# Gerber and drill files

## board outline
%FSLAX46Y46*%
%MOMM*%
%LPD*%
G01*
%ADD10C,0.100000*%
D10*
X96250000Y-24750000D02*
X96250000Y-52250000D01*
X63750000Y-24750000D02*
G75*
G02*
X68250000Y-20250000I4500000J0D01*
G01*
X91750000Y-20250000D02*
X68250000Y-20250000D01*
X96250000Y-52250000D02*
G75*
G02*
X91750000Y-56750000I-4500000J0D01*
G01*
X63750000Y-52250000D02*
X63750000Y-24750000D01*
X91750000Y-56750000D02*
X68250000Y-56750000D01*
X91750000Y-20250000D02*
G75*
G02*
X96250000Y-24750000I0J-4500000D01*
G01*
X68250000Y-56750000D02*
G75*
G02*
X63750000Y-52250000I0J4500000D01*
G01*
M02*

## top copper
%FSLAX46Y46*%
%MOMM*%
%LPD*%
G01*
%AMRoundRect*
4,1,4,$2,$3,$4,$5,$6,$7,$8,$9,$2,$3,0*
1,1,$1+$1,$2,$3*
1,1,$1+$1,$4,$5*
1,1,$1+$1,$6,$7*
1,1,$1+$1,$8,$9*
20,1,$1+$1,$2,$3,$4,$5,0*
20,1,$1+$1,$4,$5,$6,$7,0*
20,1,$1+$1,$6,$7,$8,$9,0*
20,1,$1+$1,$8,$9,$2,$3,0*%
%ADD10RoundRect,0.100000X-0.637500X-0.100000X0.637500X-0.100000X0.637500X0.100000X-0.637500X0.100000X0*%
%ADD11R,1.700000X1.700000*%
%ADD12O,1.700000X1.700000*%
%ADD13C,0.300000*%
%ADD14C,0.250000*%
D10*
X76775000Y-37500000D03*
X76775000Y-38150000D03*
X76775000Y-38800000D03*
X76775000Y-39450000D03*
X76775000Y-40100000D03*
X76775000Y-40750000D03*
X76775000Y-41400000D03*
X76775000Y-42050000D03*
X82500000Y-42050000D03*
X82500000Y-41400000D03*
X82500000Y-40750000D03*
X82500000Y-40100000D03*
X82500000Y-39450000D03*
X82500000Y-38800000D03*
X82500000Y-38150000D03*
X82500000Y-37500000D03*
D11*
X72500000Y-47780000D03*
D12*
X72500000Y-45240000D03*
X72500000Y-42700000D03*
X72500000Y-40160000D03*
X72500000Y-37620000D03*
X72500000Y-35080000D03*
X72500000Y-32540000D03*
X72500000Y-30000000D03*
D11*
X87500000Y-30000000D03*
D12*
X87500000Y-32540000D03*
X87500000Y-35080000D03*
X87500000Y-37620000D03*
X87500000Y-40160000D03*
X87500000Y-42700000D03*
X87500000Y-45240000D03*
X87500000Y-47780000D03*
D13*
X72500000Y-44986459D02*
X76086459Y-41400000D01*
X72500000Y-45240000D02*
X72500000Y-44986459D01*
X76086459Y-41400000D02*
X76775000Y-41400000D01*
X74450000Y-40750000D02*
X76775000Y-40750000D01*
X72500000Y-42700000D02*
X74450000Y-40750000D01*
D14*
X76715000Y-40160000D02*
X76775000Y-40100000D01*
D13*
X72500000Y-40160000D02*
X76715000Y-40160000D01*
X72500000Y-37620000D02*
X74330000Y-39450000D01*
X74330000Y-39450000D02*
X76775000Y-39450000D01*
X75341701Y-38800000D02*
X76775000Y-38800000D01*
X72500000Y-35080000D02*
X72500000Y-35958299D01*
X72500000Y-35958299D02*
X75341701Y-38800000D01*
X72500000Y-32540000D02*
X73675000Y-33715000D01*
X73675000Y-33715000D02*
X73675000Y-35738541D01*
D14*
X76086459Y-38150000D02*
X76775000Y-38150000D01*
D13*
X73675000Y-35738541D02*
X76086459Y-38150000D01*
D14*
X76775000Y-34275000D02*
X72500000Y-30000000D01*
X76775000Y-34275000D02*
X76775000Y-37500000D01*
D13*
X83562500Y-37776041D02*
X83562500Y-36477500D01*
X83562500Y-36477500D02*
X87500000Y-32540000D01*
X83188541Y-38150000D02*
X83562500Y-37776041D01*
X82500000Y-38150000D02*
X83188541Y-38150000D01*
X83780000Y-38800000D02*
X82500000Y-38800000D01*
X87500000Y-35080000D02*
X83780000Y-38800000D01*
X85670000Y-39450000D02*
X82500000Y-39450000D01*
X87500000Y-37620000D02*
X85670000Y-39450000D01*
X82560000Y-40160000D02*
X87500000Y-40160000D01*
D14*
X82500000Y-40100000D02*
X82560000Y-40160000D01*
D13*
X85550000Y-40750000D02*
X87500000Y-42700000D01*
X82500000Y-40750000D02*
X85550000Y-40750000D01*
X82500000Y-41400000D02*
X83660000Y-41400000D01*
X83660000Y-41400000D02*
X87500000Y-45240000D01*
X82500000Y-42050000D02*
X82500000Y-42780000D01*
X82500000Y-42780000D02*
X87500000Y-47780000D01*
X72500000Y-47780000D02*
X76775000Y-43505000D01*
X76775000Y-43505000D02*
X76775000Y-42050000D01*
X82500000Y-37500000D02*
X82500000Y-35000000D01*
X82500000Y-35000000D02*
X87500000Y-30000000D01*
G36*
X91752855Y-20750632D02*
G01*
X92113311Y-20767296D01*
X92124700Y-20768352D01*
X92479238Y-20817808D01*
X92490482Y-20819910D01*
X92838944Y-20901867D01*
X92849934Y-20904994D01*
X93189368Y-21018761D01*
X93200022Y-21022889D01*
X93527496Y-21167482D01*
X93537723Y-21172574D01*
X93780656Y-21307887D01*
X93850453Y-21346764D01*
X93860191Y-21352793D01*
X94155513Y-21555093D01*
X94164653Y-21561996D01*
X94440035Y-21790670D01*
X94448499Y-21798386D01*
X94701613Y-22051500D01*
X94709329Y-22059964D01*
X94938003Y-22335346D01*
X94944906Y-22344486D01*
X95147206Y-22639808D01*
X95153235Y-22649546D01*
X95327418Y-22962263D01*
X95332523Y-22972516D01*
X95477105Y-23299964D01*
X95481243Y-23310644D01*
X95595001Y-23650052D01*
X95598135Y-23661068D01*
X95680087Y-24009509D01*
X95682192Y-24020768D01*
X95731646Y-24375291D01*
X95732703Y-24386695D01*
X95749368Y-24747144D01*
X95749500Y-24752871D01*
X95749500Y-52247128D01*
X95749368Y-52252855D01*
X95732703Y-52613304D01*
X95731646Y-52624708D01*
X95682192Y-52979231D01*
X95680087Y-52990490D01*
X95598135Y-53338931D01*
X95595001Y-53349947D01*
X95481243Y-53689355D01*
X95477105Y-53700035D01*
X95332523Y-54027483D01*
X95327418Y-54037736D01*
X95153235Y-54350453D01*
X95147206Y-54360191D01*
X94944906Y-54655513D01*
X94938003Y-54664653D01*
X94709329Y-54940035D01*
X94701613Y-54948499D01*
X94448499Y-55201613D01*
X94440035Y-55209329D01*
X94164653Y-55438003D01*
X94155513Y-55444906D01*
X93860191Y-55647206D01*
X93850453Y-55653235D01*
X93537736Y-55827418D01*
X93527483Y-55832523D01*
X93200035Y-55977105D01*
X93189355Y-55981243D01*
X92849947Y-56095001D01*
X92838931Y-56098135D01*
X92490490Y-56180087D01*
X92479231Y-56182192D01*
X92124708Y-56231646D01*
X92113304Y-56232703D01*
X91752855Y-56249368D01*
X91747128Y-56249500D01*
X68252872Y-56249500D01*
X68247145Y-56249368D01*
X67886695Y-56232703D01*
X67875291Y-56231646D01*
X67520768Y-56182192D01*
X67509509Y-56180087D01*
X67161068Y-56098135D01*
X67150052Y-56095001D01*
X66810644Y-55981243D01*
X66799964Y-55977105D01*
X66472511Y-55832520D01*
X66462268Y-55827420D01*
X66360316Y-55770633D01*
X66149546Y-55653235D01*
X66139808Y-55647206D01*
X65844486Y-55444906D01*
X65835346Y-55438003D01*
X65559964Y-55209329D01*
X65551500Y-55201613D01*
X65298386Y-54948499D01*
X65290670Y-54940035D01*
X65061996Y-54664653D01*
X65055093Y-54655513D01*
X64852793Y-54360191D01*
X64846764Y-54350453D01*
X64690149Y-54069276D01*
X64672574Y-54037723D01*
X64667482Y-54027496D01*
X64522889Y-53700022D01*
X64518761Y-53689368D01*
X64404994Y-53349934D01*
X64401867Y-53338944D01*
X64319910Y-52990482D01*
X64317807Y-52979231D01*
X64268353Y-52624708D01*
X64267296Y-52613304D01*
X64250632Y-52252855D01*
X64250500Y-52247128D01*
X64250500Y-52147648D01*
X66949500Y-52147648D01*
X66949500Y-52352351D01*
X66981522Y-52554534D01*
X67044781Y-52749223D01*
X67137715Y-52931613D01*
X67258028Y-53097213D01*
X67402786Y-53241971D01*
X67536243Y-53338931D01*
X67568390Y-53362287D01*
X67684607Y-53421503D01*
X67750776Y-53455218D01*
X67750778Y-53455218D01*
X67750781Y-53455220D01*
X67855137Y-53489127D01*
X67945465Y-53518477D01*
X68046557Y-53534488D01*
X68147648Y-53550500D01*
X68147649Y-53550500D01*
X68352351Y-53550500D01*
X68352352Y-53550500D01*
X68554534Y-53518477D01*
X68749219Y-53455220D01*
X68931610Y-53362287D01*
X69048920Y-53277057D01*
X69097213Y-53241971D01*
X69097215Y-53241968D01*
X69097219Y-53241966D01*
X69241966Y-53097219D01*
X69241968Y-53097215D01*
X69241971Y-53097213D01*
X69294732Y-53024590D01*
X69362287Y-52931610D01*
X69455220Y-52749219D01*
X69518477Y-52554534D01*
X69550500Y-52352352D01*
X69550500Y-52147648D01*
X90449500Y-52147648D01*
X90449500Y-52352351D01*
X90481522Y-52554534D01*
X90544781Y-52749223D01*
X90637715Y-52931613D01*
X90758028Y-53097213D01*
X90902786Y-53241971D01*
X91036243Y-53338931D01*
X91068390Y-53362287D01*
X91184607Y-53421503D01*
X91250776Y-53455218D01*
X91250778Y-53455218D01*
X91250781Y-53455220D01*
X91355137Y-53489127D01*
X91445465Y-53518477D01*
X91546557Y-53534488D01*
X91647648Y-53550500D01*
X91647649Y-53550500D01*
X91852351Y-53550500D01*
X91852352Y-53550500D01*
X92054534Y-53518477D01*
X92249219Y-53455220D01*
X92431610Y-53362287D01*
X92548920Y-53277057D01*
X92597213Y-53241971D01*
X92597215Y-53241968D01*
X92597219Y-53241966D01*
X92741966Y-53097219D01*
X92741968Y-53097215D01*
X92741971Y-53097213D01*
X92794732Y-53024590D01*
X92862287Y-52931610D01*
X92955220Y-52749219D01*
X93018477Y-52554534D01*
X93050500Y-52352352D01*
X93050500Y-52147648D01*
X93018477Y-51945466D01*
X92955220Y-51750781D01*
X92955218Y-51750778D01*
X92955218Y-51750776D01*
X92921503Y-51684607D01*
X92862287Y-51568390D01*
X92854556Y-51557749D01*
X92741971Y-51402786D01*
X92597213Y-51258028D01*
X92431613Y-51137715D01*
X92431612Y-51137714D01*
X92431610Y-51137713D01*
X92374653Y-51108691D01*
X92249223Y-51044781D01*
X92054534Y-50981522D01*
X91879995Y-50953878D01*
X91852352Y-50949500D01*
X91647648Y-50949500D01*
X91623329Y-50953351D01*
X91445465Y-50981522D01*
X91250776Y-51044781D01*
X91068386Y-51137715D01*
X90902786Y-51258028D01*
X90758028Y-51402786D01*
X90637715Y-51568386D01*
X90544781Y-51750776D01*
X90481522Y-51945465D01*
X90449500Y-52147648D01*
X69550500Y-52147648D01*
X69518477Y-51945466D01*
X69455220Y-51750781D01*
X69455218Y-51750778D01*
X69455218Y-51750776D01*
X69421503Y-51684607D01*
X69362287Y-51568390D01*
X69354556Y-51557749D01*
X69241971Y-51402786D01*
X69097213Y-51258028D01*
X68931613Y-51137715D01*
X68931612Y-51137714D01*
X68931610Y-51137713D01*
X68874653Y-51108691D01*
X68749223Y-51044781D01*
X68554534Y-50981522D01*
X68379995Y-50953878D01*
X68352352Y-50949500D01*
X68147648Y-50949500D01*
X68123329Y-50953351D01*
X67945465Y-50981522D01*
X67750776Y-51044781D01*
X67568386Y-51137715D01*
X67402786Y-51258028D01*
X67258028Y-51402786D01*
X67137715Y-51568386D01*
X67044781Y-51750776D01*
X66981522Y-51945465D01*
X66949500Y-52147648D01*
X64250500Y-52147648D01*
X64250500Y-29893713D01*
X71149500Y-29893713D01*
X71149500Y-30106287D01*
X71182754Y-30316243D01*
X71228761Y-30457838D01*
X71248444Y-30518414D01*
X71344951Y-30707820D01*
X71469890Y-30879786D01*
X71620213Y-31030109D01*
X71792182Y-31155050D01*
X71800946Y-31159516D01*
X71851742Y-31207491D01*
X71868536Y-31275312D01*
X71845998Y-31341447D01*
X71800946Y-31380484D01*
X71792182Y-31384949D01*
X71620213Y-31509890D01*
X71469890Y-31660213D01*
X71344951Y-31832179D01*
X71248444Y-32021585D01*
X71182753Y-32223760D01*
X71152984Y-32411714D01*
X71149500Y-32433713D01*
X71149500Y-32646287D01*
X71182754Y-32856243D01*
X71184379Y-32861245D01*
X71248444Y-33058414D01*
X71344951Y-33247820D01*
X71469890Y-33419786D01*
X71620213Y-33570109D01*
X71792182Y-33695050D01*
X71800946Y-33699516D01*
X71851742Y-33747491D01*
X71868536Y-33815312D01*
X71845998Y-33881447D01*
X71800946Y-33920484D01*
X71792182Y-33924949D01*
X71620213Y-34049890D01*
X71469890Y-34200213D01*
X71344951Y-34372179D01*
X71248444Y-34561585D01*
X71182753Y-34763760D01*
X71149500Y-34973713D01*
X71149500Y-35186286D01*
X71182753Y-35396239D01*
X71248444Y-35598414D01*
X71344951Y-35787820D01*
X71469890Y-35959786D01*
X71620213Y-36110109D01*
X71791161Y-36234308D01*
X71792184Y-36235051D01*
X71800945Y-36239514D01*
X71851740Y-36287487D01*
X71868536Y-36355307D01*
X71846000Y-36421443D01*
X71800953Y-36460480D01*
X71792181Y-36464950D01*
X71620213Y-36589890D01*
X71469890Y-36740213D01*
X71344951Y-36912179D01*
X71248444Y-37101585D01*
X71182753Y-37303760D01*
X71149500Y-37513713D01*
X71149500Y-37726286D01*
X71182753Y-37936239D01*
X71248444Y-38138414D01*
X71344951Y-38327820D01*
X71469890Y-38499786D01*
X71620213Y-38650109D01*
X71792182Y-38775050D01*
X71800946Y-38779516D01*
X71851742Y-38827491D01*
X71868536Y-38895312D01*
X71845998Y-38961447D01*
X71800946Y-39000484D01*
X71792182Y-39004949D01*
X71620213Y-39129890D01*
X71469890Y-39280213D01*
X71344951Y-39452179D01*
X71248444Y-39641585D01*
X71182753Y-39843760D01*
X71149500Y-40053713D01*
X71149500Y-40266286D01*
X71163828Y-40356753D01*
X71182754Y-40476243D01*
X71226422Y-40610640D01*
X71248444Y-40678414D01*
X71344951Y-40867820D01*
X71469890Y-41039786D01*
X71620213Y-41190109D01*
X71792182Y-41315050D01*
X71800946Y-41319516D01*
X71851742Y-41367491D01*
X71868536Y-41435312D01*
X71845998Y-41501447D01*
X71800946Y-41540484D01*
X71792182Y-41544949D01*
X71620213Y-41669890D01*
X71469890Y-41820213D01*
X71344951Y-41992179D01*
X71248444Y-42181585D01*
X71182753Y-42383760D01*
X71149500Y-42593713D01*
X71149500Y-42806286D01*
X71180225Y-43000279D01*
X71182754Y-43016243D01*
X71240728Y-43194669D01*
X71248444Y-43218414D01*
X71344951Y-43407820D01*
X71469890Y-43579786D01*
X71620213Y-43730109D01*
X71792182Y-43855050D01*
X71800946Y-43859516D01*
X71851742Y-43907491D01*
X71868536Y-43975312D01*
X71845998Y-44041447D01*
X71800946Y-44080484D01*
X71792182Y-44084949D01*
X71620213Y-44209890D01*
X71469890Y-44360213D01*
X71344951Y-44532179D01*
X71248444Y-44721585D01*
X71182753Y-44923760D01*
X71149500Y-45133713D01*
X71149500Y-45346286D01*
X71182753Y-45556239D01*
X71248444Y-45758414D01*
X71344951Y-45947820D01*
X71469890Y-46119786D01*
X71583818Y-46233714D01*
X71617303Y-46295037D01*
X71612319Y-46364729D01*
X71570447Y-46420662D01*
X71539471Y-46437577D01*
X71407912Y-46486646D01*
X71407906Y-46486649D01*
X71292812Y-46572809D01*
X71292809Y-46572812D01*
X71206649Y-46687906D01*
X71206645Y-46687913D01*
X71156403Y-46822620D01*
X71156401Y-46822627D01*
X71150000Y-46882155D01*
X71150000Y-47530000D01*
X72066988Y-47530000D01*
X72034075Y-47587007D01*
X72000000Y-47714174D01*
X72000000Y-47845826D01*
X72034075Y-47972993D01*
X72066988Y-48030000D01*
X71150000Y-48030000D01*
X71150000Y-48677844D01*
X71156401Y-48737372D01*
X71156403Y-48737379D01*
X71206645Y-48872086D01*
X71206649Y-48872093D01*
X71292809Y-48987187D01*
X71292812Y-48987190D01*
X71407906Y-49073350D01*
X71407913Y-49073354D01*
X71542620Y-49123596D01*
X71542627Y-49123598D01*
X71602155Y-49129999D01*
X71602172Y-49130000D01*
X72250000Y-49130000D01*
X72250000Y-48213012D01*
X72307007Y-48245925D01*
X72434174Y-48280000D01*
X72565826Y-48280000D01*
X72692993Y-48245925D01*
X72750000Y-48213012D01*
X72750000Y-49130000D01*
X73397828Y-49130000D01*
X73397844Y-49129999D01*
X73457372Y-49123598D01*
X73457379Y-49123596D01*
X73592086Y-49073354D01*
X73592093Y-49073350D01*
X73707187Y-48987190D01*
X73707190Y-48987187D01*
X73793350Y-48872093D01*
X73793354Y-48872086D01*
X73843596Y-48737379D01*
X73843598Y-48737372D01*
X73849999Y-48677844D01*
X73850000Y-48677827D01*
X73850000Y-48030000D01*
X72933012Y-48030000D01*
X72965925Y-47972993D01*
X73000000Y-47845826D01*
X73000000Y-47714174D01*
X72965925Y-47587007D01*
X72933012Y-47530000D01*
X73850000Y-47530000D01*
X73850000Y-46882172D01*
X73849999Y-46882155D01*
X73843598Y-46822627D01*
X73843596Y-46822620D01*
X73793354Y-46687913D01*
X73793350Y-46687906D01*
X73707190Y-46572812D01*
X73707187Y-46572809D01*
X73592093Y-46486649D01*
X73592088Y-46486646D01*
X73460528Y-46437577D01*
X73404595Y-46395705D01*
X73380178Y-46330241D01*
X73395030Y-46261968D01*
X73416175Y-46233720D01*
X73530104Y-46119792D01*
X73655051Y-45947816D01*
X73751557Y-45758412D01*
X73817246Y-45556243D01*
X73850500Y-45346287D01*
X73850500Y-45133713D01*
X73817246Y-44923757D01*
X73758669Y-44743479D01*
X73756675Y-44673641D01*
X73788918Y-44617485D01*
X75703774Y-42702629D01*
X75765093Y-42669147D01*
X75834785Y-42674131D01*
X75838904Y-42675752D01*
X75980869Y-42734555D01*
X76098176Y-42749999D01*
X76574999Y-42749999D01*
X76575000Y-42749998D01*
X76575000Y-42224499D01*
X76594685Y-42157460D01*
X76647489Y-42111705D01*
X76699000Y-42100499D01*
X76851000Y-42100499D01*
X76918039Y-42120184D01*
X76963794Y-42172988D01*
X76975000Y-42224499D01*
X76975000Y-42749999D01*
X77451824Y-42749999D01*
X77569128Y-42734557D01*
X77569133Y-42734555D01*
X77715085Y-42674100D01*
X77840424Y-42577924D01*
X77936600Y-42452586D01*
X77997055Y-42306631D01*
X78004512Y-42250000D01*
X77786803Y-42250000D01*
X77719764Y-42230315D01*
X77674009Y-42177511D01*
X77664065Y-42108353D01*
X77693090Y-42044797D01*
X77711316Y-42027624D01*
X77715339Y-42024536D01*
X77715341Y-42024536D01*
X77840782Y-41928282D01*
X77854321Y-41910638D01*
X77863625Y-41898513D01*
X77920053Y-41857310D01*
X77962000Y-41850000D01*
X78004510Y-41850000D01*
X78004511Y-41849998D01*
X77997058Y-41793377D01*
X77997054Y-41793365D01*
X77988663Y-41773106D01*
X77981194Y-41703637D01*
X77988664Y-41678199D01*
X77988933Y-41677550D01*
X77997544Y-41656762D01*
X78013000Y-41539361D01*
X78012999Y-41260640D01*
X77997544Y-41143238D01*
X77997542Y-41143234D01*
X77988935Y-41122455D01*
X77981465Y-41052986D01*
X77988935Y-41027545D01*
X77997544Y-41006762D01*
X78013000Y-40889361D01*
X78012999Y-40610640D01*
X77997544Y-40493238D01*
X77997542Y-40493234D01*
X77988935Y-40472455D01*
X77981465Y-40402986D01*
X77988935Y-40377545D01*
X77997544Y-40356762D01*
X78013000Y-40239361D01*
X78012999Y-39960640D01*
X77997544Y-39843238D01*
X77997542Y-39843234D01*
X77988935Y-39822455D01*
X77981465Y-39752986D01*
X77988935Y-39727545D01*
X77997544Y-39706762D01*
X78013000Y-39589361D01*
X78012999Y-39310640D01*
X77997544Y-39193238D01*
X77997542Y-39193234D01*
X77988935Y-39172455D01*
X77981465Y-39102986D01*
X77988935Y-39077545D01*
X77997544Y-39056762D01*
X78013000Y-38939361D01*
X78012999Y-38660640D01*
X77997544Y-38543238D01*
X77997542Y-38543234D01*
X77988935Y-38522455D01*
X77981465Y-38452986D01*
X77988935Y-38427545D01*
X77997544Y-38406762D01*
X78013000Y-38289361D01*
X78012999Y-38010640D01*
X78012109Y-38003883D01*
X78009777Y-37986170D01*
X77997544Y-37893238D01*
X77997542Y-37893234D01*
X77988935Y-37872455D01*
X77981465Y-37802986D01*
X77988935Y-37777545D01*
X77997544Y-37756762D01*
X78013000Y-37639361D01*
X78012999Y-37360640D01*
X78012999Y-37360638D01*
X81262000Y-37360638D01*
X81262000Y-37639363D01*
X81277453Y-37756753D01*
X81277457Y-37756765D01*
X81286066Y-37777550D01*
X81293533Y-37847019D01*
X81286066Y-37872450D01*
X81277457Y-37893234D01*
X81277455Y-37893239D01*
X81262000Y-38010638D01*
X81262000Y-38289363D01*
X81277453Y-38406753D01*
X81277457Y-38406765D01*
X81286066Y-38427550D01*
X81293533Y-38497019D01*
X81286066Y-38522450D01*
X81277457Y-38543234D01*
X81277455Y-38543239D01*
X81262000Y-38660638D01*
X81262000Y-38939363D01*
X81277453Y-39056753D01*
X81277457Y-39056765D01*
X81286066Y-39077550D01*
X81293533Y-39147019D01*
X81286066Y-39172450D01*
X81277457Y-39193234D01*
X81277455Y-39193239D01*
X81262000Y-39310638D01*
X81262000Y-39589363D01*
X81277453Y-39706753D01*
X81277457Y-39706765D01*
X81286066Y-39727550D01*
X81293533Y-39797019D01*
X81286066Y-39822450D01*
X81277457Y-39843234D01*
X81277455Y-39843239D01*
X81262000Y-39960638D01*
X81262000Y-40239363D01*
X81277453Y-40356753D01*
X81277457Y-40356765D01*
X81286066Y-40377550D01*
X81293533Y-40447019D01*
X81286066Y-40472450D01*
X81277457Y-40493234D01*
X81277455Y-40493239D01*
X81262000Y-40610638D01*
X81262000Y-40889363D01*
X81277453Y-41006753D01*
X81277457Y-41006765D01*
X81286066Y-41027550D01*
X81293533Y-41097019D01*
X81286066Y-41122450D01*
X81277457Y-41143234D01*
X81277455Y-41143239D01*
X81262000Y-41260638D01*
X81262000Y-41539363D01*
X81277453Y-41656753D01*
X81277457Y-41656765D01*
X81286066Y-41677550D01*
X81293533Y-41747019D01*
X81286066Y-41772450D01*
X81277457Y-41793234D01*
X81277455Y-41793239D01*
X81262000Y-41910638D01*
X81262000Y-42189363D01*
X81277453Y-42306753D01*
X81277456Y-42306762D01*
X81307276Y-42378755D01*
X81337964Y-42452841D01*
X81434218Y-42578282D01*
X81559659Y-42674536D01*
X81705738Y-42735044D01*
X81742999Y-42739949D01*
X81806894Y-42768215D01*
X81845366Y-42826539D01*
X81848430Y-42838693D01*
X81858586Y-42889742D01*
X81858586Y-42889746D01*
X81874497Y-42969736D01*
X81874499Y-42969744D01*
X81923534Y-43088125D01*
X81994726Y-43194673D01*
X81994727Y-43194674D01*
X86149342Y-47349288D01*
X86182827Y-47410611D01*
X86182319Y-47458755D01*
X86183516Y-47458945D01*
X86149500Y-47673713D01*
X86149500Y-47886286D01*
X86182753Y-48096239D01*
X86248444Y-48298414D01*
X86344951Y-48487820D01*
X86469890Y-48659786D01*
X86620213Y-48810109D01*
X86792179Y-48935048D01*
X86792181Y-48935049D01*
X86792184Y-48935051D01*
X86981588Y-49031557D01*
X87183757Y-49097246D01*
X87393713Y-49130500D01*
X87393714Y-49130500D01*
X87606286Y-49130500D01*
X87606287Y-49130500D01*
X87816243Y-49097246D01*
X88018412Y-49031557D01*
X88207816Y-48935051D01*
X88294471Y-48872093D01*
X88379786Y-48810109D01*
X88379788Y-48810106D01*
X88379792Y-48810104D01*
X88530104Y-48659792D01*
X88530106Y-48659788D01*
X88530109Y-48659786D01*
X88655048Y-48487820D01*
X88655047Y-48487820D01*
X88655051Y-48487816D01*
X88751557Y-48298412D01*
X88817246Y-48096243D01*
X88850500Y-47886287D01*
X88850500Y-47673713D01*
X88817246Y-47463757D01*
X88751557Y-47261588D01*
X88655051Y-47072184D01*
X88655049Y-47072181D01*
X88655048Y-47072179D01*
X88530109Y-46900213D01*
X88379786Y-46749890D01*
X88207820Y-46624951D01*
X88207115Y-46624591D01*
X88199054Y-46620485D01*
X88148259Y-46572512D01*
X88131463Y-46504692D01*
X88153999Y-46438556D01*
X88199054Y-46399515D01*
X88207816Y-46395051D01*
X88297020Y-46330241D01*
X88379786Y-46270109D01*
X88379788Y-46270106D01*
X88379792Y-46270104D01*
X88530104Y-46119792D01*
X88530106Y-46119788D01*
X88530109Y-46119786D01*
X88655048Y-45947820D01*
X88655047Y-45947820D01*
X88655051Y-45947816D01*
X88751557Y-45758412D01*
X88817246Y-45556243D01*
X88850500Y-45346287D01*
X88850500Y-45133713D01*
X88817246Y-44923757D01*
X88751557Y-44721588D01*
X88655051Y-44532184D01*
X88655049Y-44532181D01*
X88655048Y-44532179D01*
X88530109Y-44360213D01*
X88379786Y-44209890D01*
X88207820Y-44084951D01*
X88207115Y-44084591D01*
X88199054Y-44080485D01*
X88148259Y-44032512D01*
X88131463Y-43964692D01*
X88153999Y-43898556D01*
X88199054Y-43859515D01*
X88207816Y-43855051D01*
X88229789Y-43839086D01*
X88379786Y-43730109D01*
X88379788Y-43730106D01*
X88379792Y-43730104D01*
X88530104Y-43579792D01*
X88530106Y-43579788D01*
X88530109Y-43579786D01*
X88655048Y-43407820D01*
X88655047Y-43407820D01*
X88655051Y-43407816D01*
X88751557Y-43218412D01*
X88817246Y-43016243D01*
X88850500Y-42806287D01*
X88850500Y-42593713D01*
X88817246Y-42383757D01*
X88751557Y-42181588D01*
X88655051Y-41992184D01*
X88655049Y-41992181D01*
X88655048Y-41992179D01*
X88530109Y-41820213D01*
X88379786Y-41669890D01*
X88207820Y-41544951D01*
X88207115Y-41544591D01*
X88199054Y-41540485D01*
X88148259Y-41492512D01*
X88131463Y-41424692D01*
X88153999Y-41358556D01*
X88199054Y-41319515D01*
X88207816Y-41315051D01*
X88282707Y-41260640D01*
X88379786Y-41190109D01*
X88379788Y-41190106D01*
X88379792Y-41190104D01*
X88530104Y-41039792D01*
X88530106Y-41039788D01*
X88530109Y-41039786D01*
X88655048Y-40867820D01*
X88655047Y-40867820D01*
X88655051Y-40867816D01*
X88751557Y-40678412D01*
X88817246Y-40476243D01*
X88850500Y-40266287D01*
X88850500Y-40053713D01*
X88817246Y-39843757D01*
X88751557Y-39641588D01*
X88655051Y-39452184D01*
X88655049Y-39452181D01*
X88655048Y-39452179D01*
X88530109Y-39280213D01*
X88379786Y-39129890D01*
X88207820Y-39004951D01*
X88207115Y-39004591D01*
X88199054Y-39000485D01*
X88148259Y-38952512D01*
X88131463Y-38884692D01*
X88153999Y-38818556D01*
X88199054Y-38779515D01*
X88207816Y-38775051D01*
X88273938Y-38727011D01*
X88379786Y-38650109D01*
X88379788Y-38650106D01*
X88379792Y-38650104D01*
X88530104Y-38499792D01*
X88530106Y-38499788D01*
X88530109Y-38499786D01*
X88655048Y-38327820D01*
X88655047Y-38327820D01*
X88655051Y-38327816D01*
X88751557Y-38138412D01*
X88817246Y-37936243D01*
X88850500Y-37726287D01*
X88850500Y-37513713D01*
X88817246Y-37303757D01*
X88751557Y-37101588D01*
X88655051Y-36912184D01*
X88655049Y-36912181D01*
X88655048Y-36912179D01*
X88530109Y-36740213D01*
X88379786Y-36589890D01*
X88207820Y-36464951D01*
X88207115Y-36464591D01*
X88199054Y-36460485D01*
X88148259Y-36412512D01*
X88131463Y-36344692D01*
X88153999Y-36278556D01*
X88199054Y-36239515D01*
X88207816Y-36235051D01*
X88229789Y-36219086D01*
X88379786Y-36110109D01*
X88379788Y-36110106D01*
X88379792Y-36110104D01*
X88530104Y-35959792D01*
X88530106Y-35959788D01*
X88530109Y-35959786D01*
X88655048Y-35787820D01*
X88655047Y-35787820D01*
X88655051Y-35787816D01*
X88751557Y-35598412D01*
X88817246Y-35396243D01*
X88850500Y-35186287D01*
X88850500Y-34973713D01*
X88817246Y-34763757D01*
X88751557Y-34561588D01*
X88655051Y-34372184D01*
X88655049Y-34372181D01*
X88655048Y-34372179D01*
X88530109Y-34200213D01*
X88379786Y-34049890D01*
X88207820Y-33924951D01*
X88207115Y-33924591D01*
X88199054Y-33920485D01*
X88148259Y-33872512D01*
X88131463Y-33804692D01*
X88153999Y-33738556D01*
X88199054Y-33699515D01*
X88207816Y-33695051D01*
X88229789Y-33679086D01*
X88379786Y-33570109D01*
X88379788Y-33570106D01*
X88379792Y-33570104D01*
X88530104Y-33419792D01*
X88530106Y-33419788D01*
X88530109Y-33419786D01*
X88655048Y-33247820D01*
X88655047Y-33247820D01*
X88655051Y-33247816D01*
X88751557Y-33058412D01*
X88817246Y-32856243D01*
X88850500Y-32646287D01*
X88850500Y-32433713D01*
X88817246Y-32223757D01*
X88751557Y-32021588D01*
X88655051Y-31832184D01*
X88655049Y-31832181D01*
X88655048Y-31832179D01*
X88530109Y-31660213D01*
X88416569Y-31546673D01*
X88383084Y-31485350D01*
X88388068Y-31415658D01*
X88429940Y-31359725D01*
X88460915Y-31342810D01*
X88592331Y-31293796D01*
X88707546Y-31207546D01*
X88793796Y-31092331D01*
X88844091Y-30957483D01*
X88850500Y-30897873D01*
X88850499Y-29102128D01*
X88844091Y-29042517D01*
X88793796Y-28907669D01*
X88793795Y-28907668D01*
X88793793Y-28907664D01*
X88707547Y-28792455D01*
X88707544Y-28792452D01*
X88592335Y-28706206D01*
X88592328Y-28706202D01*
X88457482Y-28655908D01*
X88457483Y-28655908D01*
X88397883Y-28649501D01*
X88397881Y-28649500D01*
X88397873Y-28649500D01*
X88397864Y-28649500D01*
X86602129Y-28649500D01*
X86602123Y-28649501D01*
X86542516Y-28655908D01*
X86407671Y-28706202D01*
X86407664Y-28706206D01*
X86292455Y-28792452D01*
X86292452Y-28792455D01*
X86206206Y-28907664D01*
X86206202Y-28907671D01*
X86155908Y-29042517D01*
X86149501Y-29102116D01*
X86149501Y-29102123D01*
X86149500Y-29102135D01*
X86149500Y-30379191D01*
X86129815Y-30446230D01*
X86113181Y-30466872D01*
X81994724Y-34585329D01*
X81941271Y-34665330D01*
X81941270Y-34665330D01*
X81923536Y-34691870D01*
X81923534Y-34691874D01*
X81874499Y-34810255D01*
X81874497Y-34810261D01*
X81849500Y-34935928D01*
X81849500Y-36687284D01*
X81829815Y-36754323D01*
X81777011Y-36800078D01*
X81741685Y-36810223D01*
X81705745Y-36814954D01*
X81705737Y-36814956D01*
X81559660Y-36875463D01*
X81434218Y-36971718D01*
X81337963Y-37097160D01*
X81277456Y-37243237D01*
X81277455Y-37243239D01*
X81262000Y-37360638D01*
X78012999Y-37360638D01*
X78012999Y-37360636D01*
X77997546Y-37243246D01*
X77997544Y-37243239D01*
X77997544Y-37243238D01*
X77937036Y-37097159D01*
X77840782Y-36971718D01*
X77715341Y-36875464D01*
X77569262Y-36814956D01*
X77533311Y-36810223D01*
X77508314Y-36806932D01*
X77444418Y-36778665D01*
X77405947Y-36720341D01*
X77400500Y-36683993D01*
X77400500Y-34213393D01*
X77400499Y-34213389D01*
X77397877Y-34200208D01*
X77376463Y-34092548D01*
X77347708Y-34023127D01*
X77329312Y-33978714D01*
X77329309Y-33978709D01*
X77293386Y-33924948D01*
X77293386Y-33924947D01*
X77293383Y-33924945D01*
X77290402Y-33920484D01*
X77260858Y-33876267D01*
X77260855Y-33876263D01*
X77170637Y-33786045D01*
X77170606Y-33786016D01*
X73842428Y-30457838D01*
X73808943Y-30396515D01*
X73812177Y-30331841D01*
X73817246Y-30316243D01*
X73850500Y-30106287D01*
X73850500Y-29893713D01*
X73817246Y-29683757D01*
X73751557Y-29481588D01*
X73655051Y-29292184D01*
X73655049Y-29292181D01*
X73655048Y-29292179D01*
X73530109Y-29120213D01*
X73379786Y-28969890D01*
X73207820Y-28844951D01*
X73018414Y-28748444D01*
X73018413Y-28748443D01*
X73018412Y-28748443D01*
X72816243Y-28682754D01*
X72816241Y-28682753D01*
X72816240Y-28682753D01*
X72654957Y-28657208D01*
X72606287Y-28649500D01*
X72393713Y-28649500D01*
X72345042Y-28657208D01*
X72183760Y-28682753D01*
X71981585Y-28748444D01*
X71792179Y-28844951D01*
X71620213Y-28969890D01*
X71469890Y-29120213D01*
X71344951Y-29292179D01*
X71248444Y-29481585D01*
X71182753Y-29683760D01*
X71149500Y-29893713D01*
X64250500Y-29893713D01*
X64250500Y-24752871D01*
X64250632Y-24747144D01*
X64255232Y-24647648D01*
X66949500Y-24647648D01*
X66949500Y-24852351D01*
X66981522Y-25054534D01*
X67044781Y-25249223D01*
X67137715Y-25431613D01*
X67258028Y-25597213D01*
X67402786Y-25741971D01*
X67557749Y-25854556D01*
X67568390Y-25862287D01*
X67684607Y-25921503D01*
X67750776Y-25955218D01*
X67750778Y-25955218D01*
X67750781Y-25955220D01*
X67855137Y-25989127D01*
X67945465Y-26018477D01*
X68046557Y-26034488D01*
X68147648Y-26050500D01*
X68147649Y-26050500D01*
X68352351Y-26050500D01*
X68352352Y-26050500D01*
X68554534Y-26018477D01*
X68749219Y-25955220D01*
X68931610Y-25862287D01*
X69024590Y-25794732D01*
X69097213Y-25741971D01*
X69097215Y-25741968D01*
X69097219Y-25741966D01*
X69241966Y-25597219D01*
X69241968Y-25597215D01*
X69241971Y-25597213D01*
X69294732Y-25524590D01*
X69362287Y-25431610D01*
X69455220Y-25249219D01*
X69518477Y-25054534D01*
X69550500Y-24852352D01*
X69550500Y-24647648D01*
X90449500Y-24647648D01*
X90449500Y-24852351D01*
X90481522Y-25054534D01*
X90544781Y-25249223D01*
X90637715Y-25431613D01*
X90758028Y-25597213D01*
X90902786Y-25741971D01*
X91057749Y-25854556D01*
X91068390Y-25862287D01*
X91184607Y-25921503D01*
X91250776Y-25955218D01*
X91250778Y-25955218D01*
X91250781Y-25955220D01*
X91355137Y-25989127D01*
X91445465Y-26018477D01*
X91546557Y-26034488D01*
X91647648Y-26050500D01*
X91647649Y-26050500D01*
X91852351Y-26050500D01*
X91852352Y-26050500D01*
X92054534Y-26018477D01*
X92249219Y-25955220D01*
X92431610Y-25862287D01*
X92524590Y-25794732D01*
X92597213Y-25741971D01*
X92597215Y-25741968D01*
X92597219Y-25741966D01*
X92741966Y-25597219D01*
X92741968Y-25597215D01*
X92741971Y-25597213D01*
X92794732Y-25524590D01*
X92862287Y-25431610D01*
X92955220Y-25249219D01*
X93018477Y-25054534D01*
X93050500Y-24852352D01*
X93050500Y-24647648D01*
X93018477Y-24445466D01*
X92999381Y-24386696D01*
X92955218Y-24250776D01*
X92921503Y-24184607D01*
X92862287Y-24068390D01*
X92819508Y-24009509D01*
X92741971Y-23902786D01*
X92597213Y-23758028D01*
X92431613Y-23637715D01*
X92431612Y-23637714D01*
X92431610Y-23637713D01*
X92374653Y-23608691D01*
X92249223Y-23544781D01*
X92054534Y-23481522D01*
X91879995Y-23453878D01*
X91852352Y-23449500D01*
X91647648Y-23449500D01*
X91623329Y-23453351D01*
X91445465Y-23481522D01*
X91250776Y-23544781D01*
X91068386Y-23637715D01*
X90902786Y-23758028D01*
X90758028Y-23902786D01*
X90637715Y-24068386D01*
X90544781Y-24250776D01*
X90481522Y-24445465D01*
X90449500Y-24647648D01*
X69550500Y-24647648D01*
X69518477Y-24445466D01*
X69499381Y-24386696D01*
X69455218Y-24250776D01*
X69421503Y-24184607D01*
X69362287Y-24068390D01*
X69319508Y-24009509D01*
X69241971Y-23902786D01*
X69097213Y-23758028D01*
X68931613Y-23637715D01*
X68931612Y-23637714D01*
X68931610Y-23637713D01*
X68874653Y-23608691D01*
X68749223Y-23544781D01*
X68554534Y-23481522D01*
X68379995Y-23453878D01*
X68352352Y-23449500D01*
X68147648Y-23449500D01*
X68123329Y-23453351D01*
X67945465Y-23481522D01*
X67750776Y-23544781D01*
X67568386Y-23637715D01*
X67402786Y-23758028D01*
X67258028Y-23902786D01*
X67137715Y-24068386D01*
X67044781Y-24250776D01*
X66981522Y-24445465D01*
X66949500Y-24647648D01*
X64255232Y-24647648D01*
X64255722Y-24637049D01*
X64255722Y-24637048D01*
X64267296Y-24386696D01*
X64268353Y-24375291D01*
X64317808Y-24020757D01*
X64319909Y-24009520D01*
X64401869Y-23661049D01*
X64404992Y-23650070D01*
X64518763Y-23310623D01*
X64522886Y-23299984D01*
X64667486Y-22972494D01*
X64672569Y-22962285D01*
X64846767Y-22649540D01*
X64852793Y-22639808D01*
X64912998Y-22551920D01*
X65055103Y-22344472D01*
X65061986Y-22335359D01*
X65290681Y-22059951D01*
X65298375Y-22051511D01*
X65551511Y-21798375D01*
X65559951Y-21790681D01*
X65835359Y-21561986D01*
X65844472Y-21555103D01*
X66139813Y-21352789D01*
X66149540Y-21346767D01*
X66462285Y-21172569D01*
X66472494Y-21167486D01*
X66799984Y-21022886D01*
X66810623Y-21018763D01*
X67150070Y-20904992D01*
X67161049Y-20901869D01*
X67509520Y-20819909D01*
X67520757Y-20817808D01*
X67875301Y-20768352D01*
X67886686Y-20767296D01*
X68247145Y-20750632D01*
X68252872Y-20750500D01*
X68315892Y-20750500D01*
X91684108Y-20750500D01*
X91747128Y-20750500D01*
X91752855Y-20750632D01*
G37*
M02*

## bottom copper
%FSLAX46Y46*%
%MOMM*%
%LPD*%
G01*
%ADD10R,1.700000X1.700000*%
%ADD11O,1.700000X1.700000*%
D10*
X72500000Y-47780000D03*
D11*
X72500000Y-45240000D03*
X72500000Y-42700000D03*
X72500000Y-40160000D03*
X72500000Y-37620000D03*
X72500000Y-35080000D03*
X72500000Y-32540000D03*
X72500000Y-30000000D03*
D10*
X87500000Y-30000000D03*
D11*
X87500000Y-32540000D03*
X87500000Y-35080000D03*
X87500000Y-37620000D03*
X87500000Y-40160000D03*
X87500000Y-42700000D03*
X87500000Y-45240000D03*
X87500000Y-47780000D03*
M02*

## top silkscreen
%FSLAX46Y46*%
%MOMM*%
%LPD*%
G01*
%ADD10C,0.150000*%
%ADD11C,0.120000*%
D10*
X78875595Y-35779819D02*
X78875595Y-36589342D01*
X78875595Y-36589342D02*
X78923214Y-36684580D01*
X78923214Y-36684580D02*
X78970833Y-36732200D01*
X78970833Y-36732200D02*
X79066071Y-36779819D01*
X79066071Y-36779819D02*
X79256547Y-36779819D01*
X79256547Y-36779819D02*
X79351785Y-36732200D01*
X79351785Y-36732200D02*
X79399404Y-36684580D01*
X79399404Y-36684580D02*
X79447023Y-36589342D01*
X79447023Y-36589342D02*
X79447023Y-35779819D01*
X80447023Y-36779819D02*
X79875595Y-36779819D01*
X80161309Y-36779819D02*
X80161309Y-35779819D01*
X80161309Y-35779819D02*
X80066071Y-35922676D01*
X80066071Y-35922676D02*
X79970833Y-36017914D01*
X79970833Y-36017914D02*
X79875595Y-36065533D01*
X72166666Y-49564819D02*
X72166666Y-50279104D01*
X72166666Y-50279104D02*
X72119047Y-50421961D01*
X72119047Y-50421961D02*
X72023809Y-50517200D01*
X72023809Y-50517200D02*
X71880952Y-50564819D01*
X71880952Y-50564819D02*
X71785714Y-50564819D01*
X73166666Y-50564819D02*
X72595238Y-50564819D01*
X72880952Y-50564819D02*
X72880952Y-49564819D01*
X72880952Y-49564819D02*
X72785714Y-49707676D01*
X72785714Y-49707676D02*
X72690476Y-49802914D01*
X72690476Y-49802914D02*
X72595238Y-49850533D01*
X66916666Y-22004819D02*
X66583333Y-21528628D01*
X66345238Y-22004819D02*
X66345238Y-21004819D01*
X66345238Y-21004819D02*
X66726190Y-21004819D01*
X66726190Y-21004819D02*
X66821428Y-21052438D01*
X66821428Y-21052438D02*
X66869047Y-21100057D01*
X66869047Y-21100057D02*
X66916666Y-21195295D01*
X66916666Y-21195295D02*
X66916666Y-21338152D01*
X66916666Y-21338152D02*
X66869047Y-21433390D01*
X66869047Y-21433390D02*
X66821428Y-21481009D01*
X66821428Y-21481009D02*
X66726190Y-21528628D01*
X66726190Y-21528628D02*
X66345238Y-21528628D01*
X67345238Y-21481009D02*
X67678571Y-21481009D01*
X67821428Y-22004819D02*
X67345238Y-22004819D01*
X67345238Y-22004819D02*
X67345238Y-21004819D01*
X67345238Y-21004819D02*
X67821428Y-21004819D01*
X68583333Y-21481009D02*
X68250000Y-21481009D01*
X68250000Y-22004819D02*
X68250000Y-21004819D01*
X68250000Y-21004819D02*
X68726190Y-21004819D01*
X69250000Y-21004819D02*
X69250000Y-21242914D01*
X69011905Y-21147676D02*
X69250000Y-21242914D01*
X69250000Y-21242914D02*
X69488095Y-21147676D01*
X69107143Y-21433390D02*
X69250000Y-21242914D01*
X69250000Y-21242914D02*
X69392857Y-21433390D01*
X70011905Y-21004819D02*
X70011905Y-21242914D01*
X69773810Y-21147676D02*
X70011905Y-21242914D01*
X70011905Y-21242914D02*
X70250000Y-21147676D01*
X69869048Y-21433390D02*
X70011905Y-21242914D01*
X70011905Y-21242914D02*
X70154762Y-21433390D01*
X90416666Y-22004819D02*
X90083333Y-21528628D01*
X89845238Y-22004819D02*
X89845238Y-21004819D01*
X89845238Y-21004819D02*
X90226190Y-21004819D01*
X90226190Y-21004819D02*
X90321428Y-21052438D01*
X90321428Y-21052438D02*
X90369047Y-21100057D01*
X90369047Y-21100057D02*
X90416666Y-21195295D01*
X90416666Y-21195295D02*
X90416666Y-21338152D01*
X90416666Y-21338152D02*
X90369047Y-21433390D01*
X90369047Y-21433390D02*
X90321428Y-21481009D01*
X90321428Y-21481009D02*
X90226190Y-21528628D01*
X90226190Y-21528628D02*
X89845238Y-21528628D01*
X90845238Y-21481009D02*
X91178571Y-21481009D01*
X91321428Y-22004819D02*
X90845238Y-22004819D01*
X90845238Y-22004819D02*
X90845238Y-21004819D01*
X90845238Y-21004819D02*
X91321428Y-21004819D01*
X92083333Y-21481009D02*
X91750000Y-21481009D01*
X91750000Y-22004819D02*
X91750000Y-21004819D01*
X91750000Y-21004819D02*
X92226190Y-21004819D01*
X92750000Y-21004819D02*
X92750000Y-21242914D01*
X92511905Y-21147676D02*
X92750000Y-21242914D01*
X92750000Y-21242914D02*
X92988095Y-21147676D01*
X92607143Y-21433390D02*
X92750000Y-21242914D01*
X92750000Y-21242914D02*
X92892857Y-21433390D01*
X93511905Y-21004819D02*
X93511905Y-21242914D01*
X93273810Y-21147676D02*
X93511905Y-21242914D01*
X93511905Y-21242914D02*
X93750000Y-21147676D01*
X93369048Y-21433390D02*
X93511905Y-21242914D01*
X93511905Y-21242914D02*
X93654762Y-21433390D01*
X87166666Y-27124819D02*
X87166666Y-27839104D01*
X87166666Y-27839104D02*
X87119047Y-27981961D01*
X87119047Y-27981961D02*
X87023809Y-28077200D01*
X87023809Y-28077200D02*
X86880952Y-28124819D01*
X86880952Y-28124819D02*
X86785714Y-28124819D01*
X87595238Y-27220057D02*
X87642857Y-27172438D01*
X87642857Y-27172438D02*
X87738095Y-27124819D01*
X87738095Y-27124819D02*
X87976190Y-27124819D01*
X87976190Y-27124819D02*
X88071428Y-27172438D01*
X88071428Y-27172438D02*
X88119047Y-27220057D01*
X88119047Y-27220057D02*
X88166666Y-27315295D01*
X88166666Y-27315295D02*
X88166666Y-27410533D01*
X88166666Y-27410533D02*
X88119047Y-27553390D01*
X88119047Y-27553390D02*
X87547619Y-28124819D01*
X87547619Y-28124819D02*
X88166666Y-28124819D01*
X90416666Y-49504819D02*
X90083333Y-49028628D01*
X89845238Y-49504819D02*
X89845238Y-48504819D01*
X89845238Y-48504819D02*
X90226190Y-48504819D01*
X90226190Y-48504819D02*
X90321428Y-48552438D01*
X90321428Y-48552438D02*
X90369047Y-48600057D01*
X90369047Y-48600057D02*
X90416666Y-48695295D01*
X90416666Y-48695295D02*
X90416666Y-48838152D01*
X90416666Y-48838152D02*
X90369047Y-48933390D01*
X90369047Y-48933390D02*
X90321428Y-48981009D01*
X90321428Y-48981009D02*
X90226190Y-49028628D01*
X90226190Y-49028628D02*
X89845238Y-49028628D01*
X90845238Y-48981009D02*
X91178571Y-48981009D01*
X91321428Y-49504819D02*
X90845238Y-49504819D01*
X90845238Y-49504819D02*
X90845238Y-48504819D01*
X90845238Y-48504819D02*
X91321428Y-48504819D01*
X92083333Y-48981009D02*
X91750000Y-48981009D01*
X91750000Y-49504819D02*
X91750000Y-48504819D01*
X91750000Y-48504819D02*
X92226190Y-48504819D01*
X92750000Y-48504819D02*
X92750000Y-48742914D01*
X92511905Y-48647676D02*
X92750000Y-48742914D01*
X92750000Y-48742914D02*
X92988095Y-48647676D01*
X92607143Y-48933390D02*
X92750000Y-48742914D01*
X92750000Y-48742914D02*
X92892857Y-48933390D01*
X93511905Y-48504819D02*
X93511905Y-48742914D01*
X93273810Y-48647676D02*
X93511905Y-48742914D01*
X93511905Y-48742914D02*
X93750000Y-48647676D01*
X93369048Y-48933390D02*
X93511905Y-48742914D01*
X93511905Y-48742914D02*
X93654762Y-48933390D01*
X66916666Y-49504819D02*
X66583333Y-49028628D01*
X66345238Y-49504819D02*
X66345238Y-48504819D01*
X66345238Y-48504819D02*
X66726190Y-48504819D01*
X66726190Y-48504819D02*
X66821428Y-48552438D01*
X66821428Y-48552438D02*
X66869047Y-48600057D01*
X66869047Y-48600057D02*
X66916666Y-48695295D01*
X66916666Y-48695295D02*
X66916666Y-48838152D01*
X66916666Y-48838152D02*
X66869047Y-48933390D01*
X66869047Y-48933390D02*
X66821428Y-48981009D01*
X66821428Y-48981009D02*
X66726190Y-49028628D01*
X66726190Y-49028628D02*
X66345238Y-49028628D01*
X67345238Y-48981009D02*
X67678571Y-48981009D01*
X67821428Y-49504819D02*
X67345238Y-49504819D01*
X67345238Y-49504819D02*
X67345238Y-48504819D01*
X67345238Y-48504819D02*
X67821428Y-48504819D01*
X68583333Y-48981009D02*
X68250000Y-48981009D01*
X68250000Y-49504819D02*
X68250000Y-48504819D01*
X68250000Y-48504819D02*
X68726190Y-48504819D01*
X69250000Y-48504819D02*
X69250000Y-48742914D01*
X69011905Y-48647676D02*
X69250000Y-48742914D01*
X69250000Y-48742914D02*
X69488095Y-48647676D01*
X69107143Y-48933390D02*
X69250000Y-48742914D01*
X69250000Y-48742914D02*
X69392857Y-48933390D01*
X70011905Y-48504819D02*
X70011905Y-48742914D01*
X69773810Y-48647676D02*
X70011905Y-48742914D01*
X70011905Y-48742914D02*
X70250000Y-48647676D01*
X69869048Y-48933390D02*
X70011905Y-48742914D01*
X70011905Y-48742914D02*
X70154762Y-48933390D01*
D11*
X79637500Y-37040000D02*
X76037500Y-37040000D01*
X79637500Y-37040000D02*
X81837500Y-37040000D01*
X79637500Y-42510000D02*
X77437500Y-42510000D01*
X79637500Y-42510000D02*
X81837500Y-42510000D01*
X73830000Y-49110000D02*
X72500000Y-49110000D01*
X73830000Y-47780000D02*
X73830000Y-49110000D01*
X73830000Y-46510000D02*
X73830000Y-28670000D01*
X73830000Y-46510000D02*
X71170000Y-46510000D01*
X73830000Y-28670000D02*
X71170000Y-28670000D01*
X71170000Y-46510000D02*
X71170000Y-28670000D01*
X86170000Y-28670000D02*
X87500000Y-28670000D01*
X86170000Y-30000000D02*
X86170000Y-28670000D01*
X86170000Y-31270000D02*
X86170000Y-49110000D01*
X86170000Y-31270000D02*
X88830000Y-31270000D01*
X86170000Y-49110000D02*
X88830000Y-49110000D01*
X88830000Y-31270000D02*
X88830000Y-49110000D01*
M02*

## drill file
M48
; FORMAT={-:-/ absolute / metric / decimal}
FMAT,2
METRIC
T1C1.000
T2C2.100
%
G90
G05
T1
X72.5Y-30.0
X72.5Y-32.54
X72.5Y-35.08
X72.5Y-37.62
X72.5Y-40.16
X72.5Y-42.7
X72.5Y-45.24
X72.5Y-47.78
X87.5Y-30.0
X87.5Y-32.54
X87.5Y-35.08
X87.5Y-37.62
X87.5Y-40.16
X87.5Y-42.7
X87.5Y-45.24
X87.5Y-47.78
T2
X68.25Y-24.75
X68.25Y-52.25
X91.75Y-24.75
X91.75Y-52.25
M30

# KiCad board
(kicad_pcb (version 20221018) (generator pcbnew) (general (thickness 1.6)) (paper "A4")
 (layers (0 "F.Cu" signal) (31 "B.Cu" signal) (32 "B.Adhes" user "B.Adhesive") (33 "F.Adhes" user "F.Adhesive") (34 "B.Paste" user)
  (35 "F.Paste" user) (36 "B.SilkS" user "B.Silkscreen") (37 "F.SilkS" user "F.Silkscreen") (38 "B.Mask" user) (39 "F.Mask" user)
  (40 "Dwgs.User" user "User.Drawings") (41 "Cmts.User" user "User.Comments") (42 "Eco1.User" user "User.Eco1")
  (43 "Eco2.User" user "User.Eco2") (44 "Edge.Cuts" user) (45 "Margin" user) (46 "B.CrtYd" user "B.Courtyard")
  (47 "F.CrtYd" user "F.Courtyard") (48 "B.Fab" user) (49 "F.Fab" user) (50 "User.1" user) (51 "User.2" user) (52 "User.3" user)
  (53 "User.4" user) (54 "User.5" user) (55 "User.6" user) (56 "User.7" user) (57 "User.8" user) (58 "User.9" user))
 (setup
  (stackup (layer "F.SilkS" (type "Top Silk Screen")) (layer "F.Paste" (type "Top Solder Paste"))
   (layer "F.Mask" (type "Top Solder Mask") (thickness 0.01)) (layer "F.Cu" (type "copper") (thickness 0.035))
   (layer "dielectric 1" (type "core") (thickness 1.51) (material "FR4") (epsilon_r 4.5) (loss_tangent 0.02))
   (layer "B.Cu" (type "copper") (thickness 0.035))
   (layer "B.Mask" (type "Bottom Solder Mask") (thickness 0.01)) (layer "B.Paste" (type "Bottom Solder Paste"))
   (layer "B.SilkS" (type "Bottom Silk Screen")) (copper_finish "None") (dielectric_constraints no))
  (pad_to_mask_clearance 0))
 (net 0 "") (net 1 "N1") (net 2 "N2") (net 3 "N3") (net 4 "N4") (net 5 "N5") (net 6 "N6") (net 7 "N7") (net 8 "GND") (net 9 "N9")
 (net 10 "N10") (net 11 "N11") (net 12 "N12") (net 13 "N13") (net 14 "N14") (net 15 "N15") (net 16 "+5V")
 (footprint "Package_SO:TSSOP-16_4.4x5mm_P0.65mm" (layer "F.Cu") (at 79.6375 39.775)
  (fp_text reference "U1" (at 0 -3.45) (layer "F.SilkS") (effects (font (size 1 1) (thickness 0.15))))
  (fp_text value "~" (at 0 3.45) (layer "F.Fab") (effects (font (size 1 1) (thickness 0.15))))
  (fp_line (start 0 -2.735) (end -3.6 -2.735) (stroke (width 0.12) (type solid)) (layer "F.SilkS"))
  (fp_line (start 0 -2.735) (end 2.2 -2.735) (stroke (width 0.12) (type solid)) (layer "F.SilkS"))
  (fp_line (start 0 2.735) (end -2.2 2.735) (stroke (width 0.12) (type solid)) (layer "F.SilkS"))
  (fp_line (start 0 2.735) (end 2.2 2.735) (stroke (width 0.12) (type solid)) (layer "F.SilkS"))
  (pad "1" smd roundrect (at -2.8625 -2.275) (size 1.475 0.4) (layers "F.Cu" "F.Paste" "F.Mask") (roundrect_rratio 0.25) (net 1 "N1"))
  (pad "2" smd roundrect (at -2.8625 -1.625) (size 1.475 0.4) (layers "F.Cu" "F.Paste" "F.Mask") (roundrect_rratio 0.25) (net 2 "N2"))
  (pad "3" smd roundrect (at -2.8625 -0.975) (size 1.475 0.4) (layers "F.Cu" "F.Paste" "F.Mask") (roundrect_rratio 0.25) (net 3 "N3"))
  (pad "4" smd roundrect (at -2.8625 -0.325) (size 1.475 0.4) (layers "F.Cu" "F.Paste" "F.Mask") (roundrect_rratio 0.25) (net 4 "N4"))
  (pad "5" smd roundrect (at -2.8625 0.325) (size 1.475 0.4) (layers "F.Cu" "F.Paste" "F.Mask") (roundrect_rratio 0.25) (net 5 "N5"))
  (pad "6" smd roundrect (at -2.8625 0.975) (size 1.475 0.4) (layers "F.Cu" "F.Paste" "F.Mask") (roundrect_rratio 0.25) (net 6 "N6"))
  (pad "7" smd roundrect (at -2.8625 1.625) (size 1.475 0.4) (layers "F.Cu" "F.Paste" "F.Mask") (roundrect_rratio 0.25) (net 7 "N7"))
  (pad "8" smd roundrect (at -2.8625 2.275) (size 1.475 0.4) (layers "F.Cu" "F.Paste" "F.Mask") (roundrect_rratio 0.25) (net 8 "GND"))
  (pad "9" smd roundrect (at 2.8625 2.275) (size 1.475 0.4) (layers "F.Cu" "F.Paste" "F.Mask") (roundrect_rratio 0.25) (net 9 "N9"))
  (pad "10" smd roundrect (at 2.8625 1.625) (size 1.475 0.4) (layers "F.Cu" "F.Paste" "F.Mask") (roundrect_rratio 0.25) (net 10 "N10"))
  (pad "11" smd roundrect (at 2.8625 0.975) (size 1.475 0.4) (layers "F.Cu" "F.Paste" "F.Mask") (roundrect_rratio 0.25) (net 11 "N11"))
  (pad "12" smd roundrect (at 2.8625 0.325) (size 1.475 0.4) (layers "F.Cu" "F.Paste" "F.Mask") (roundrect_rratio 0.25) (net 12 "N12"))
  (pad "13" smd roundrect (at 2.8625 -0.325) (size 1.475 0.4) (layers "F.Cu" "F.Paste" "F.Mask") (roundrect_rratio 0.25) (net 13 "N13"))
  (pad "14" smd roundrect (at 2.8625 -0.975) (size 1.475 0.4) (layers "F.Cu" "F.Paste" "F.Mask") (roundrect_rratio 0.25) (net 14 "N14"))
  (pad "15" smd roundrect (at 2.8625 -1.625) (size 1.475 0.4) (layers "F.Cu" "F.Paste" "F.Mask") (roundrect_rratio 0.25) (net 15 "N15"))
  (pad "16" smd roundrect (at 2.8625 -2.275) (size 1.475 0.4) (layers "F.Cu" "F.Paste" "F.Mask") (roundrect_rratio 0.25) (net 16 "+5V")))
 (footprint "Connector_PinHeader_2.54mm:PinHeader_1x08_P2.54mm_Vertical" (layer "F.Cu") (at 72.5 47.78 180)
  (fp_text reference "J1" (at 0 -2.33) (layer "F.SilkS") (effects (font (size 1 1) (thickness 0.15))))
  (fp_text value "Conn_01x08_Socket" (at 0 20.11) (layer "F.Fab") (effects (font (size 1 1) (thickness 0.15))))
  (fp_line (start -1.33 -1.33) (end 0 -1.33) (stroke (width 0.12) (type solid)) (layer "F.SilkS"))
  (fp_line (start -1.33 0) (end -1.33 -1.33) (stroke (width 0.12) (type solid)) (layer "F.SilkS"))
  (fp_line (start -1.33 1.27) (end -1.33 19.11) (stroke (width 0.12) (type solid)) (layer "F.SilkS"))
  (fp_line (start -1.33 1.27) (end 1.33 1.27) (stroke (width 0.12) (type solid)) (layer "F.SilkS"))
  (fp_line (start -1.33 19.11) (end 1.33 19.11) (stroke (width 0.12) (type solid)) (layer "F.SilkS"))
  (fp_line (start 1.33 1.27) (end 1.33 19.11) (stroke (width 0.12) (type solid)) (layer "F.SilkS"))
  (pad "1" thru_hole rect (at 0 0 180) (size 1.7 1.7) (drill 1) (layers "*.Cu" "*.Mask") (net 8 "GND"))
  (pad "2" thru_hole oval (at 0 2.54 180) (size 1.7 1.7) (drill 1) (layers "*.Cu" "*.Mask") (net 7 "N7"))
  (pad "3" thru_hole oval (at 0 5.08 180) (size 1.7 1.7) (drill 1) (layers "*.Cu" "*.Mask") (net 6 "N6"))
  (pad "4" thru_hole oval (at 0 7.62 180) (size 1.7 1.7) (drill 1) (layers "*.Cu" "*.Mask") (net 5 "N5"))
  (pad "5" thru_hole oval (at 0 10.16 180) (size 1.7 1.7) (drill 1) (layers "*.Cu" "*.Mask") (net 4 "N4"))
  (pad "6" thru_hole oval (at 0 12.7 180) (size 1.7 1.7) (drill 1) (layers "*.Cu" "*.Mask") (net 3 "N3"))
  (pad "7" thru_hole oval (at 0 15.24 180) (size 1.7 1.7) (drill 1) (layers "*.Cu" "*.Mask") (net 2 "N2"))
  (pad "8" thru_hole oval (at 0 17.78 180) (size 1.7 1.7) (drill 1) (layers "*.Cu" "*.Mask") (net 1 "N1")))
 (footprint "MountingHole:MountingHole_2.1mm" (layer "F.Cu") (at 68.25 24.75)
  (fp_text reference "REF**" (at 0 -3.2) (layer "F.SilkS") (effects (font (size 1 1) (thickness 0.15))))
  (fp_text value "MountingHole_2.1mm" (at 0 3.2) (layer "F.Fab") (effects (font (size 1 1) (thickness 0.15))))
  (pad "" np_thru_hole circle (at 0 0) (size 2.1 2.1) (drill 2.1) (layers "*.Cu" "*.Mask")))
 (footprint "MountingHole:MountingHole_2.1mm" (layer "F.Cu") (at 91.75 24.75)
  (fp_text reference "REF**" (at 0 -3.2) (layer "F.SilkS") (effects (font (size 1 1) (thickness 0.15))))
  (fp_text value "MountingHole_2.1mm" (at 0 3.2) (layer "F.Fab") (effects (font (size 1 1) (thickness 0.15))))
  (pad "" np_thru_hole circle (at 0 0) (size 2.1 2.1) (drill 2.1) (layers "*.Cu" "*.Mask")))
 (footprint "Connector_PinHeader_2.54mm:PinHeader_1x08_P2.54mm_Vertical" (layer "F.Cu") (at 87.5 30)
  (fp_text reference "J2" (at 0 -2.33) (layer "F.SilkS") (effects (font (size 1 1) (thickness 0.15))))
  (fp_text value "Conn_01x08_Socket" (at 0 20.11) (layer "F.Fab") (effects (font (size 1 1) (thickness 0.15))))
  (fp_line (start -1.33 -1.33) (end 0 -1.33) (stroke (width 0.12) (type solid)) (layer "F.SilkS"))
  (fp_line (start -1.33 0) (end -1.33 -1.33) (stroke (width 0.12) (type solid)) (layer "F.SilkS"))
  (fp_line (start -1.33 1.27) (end -1.33 19.11) (stroke (width 0.12) (type solid)) (layer "F.SilkS"))
  (fp_line (start -1.33 1.27) (end 1.33 1.27) (stroke (width 0.12) (type solid)) (layer "F.SilkS"))
  (fp_line (start -1.33 19.11) (end 1.33 19.11) (stroke (width 0.12) (type solid)) (layer "F.SilkS"))
  (fp_line (start 1.33 1.27) (end 1.33 19.11) (stroke (width 0.12) (type solid)) (layer "F.SilkS"))
  (pad "1" thru_hole rect (at 0 0) (size 1.7 1.7) (drill 1) (layers "*.Cu" "*.Mask") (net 16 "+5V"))
  (pad "2" thru_hole oval (at 0 2.54) (size 1.7 1.7) (drill 1) (layers "*.Cu" "*.Mask") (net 15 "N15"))
  (pad "3" thru_hole oval (at 0 5.08) (size 1.7 1.7) (drill 1) (layers "*.Cu" "*.Mask") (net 14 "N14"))
  (pad "4" thru_hole oval (at 0 7.62) (size 1.7 1.7) (drill 1) (layers "*.Cu" "*.Mask") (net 13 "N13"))
  (pad "5" thru_hole oval (at 0 10.16) (size 1.7 1.7) (drill 1) (layers "*.Cu" "*.Mask") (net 12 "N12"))
  (pad "6" thru_hole oval (at 0 12.7) (size 1.7 1.7) (drill 1) (layers "*.Cu" "*.Mask") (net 11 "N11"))
  (pad "7" thru_hole oval (at 0 15.24) (size 1.7 1.7) (drill 1) (layers "*.Cu" "*.Mask") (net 10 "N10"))
  (pad "8" thru_hole oval (at 0 17.78) (size 1.7 1.7) (drill 1) (layers "*.Cu" "*.Mask") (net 9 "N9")))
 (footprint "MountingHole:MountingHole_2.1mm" (layer "F.Cu") (at 91.75 52.25)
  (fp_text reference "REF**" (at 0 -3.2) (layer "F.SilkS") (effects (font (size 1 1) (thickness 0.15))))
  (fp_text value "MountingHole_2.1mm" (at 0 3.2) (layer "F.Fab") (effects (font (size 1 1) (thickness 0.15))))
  (pad "" np_thru_hole circle (at 0 0) (size 2.1 2.1) (drill 2.1) (layers "*.Cu" "*.Mask")))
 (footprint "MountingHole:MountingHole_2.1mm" (layer "F.Cu") (at 68.25 52.25)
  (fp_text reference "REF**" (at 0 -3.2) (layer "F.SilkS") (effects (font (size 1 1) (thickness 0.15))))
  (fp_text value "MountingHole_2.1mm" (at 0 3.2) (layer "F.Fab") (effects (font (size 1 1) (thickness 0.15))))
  (pad "" np_thru_hole circle (at 0 0) (size 2.1 2.1) (drill 2.1) (layers "*.Cu" "*.Mask")))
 (gr_line (start 96.25 24.75) (end 96.25 52.25) (stroke (width 0.1) (type default)) (layer "Edge.Cuts"))
 (gr_arc (start 63.75 24.75) (mid 65.068019 21.568019) (end 68.25 20.25) (stroke (width 0.1) (type default)) (layer "Edge.Cuts"))
 (gr_line (start 91.75 20.25) (end 68.25 20.25) (stroke (width 0.1) (type default)) (layer "Edge.Cuts"))
 (gr_arc (start 96.25 52.25) (mid 94.931981 55.431981) (end 91.75 56.75) (stroke (width 0.1) (type default)) (layer "Edge.Cuts"))
 (gr_line (start 63.75 52.25) (end 63.75 24.75) (stroke (width 0.1) (type default)) (layer "Edge.Cuts"))
 (gr_line (start 91.75 56.75) (end 68.25 56.75) (stroke (width 0.1) (type default)) (layer "Edge.Cuts"))
 (gr_arc (start 91.75 20.25) (mid 94.931981 21.568019) (end 96.25 24.75) (stroke (width 0.1) (type default)) (layer "Edge.Cuts"))
 (gr_arc (start 68.25 56.75) (mid 65.068019 55.431981) (end 63.75 52.25) (stroke (width 0.1) (type default)) (layer "Edge.Cuts"))
 (segment (start 72.5 44.986459) (end 76.086459 41.4) (width 0.3) (layer "F.Cu") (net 7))
 (segment (start 72.5 45.24) (end 72.5 44.986459) (width 0.3) (layer "F.Cu") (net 7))
 (segment (start 76.086459 41.4) (end 76.775 41.4) (width 0.3) (layer "F.Cu") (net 7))
 (segment (start 74.45 40.75) (end 76.775 40.75) (width 0.3) (layer "F.Cu") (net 6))
 (segment (start 72.5 42.7) (end 74.45 40.75) (width 0.3) (layer "F.Cu") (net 6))
 (segment (start 76.715 40.16) (end 76.775 40.1) (width 0.25) (layer "F.Cu") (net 5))
 (segment (start 72.5 40.16) (end 76.715 40.16) (width 0.3) (layer "F.Cu") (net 5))
 (segment (start 72.5 37.62) (end 74.33 39.45) (width 0.3) (layer "F.Cu") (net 4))
 (segment (start 74.33 39.45) (end 76.775 39.45) (width 0.3) (layer "F.Cu") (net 4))
 (segment (start 75.341701 38.8) (end 76.775 38.8) (width 0.3) (layer "F.Cu") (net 3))
 (segment (start 72.5 35.08) (end 72.5 35.958299) (width 0.3) (layer "F.Cu") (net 3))
 (segment (start 72.5 35.958299) (end 75.341701 38.8) (width 0.3) (layer "F.Cu") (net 3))
 (segment (start 72.5 32.54) (end 73.675 33.715) (width 0.3) (layer "F.Cu") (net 2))
 (segment (start 73.675 33.715) (end 73.675 35.738541) (width 0.3) (layer "F.Cu") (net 2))
 (segment (start 76.086459 38.15) (end 76.775 38.15) (width 0.25) (layer "F.Cu") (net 2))
 (segment (start 73.675 35.738541) (end 76.086459 38.15) (width 0.3) (layer "F.Cu") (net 2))
 (segment (start 76.775 34.275) (end 72.5 30) (width 0.25) (layer "F.Cu") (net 1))
 (segment (start 76.775 34.275) (end 76.775 37.5) (width 0.25) (layer "F.Cu") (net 1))
 (segment (start 83.5625 37.776041) (end 83.5625 36.4775) (width 0.3) (layer "F.Cu") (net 15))
 (segment (start 83.5625 36.4775) (end 87.5 32.54) (width 0.3) (layer "F.Cu") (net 15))
 (segment (start 83.188541 38.15) (end 83.5625 37.776041) (width 0.3) (layer "F.Cu") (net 15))
 (segment (start 82.5 38.15) (end 83.188541 38.15) (width 0.3) (layer "F.Cu") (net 15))
 (segment (start 83.78 38.8) (end 82.5 38.8) (width 0.3) (layer "F.Cu") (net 14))
 (segment (start 87.5 35.08) (end 83.78 38.8) (width 0.3) (layer "F.Cu") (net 14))
 (segment (start 85.67 39.45) (end 82.5 39.45) (width 0.3) (layer "F.Cu") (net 13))
 (segment (start 87.5 37.62) (end 85.67 39.45) (width 0.3) (layer "F.Cu") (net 13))
 (segment (start 82.56 40.16) (end 87.5 40.16) (width 0.3) (layer "F.Cu") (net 12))
 (segment (start 82.5 40.1) (end 82.56 40.16) (width 0.25) (layer "F.Cu") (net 12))
 (segment (start 85.55 40.75) (end 87.5 42.7) (width 0.3) (layer "F.Cu") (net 11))
 (segment (start 82.5 40.75) (end 85.55 40.75) (width 0.3) (layer "F.Cu") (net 11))
 (segment (start 82.5 41.4) (end 83.66 41.4) (width 0.3) (layer "F.Cu") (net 10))
 (segment (start 83.66 41.4) (end 87.5 45.24) (width 0.3) (layer "F.Cu") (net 10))
 (segment (start 82.5 42.05) (end 82.5 42.78) (width 0.3) (layer "F.Cu") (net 9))
 (segment (start 82.5 42.78) (end 87.5 47.78) (width 0.3) (layer "F.Cu") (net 9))
 (segment (start 72.5 47.78) (end 76.775 43.505) (width 0.3) (layer "F.Cu") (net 8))
 (segment (start 76.775 43.505) (end 76.775 42.05) (width 0.3) (layer "F.Cu") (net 8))
 (segment (start 82.5 37.5) (end 82.5 35) (width 0.3) (layer "F.Cu") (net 16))
 (segment (start 82.5 35) (end 87.5 30) (width 0.3) (layer "F.Cu") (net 16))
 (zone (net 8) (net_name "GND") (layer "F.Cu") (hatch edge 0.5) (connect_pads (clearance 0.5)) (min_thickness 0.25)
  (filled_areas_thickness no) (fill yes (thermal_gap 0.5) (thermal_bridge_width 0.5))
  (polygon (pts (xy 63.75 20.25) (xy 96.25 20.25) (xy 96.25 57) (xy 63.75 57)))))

